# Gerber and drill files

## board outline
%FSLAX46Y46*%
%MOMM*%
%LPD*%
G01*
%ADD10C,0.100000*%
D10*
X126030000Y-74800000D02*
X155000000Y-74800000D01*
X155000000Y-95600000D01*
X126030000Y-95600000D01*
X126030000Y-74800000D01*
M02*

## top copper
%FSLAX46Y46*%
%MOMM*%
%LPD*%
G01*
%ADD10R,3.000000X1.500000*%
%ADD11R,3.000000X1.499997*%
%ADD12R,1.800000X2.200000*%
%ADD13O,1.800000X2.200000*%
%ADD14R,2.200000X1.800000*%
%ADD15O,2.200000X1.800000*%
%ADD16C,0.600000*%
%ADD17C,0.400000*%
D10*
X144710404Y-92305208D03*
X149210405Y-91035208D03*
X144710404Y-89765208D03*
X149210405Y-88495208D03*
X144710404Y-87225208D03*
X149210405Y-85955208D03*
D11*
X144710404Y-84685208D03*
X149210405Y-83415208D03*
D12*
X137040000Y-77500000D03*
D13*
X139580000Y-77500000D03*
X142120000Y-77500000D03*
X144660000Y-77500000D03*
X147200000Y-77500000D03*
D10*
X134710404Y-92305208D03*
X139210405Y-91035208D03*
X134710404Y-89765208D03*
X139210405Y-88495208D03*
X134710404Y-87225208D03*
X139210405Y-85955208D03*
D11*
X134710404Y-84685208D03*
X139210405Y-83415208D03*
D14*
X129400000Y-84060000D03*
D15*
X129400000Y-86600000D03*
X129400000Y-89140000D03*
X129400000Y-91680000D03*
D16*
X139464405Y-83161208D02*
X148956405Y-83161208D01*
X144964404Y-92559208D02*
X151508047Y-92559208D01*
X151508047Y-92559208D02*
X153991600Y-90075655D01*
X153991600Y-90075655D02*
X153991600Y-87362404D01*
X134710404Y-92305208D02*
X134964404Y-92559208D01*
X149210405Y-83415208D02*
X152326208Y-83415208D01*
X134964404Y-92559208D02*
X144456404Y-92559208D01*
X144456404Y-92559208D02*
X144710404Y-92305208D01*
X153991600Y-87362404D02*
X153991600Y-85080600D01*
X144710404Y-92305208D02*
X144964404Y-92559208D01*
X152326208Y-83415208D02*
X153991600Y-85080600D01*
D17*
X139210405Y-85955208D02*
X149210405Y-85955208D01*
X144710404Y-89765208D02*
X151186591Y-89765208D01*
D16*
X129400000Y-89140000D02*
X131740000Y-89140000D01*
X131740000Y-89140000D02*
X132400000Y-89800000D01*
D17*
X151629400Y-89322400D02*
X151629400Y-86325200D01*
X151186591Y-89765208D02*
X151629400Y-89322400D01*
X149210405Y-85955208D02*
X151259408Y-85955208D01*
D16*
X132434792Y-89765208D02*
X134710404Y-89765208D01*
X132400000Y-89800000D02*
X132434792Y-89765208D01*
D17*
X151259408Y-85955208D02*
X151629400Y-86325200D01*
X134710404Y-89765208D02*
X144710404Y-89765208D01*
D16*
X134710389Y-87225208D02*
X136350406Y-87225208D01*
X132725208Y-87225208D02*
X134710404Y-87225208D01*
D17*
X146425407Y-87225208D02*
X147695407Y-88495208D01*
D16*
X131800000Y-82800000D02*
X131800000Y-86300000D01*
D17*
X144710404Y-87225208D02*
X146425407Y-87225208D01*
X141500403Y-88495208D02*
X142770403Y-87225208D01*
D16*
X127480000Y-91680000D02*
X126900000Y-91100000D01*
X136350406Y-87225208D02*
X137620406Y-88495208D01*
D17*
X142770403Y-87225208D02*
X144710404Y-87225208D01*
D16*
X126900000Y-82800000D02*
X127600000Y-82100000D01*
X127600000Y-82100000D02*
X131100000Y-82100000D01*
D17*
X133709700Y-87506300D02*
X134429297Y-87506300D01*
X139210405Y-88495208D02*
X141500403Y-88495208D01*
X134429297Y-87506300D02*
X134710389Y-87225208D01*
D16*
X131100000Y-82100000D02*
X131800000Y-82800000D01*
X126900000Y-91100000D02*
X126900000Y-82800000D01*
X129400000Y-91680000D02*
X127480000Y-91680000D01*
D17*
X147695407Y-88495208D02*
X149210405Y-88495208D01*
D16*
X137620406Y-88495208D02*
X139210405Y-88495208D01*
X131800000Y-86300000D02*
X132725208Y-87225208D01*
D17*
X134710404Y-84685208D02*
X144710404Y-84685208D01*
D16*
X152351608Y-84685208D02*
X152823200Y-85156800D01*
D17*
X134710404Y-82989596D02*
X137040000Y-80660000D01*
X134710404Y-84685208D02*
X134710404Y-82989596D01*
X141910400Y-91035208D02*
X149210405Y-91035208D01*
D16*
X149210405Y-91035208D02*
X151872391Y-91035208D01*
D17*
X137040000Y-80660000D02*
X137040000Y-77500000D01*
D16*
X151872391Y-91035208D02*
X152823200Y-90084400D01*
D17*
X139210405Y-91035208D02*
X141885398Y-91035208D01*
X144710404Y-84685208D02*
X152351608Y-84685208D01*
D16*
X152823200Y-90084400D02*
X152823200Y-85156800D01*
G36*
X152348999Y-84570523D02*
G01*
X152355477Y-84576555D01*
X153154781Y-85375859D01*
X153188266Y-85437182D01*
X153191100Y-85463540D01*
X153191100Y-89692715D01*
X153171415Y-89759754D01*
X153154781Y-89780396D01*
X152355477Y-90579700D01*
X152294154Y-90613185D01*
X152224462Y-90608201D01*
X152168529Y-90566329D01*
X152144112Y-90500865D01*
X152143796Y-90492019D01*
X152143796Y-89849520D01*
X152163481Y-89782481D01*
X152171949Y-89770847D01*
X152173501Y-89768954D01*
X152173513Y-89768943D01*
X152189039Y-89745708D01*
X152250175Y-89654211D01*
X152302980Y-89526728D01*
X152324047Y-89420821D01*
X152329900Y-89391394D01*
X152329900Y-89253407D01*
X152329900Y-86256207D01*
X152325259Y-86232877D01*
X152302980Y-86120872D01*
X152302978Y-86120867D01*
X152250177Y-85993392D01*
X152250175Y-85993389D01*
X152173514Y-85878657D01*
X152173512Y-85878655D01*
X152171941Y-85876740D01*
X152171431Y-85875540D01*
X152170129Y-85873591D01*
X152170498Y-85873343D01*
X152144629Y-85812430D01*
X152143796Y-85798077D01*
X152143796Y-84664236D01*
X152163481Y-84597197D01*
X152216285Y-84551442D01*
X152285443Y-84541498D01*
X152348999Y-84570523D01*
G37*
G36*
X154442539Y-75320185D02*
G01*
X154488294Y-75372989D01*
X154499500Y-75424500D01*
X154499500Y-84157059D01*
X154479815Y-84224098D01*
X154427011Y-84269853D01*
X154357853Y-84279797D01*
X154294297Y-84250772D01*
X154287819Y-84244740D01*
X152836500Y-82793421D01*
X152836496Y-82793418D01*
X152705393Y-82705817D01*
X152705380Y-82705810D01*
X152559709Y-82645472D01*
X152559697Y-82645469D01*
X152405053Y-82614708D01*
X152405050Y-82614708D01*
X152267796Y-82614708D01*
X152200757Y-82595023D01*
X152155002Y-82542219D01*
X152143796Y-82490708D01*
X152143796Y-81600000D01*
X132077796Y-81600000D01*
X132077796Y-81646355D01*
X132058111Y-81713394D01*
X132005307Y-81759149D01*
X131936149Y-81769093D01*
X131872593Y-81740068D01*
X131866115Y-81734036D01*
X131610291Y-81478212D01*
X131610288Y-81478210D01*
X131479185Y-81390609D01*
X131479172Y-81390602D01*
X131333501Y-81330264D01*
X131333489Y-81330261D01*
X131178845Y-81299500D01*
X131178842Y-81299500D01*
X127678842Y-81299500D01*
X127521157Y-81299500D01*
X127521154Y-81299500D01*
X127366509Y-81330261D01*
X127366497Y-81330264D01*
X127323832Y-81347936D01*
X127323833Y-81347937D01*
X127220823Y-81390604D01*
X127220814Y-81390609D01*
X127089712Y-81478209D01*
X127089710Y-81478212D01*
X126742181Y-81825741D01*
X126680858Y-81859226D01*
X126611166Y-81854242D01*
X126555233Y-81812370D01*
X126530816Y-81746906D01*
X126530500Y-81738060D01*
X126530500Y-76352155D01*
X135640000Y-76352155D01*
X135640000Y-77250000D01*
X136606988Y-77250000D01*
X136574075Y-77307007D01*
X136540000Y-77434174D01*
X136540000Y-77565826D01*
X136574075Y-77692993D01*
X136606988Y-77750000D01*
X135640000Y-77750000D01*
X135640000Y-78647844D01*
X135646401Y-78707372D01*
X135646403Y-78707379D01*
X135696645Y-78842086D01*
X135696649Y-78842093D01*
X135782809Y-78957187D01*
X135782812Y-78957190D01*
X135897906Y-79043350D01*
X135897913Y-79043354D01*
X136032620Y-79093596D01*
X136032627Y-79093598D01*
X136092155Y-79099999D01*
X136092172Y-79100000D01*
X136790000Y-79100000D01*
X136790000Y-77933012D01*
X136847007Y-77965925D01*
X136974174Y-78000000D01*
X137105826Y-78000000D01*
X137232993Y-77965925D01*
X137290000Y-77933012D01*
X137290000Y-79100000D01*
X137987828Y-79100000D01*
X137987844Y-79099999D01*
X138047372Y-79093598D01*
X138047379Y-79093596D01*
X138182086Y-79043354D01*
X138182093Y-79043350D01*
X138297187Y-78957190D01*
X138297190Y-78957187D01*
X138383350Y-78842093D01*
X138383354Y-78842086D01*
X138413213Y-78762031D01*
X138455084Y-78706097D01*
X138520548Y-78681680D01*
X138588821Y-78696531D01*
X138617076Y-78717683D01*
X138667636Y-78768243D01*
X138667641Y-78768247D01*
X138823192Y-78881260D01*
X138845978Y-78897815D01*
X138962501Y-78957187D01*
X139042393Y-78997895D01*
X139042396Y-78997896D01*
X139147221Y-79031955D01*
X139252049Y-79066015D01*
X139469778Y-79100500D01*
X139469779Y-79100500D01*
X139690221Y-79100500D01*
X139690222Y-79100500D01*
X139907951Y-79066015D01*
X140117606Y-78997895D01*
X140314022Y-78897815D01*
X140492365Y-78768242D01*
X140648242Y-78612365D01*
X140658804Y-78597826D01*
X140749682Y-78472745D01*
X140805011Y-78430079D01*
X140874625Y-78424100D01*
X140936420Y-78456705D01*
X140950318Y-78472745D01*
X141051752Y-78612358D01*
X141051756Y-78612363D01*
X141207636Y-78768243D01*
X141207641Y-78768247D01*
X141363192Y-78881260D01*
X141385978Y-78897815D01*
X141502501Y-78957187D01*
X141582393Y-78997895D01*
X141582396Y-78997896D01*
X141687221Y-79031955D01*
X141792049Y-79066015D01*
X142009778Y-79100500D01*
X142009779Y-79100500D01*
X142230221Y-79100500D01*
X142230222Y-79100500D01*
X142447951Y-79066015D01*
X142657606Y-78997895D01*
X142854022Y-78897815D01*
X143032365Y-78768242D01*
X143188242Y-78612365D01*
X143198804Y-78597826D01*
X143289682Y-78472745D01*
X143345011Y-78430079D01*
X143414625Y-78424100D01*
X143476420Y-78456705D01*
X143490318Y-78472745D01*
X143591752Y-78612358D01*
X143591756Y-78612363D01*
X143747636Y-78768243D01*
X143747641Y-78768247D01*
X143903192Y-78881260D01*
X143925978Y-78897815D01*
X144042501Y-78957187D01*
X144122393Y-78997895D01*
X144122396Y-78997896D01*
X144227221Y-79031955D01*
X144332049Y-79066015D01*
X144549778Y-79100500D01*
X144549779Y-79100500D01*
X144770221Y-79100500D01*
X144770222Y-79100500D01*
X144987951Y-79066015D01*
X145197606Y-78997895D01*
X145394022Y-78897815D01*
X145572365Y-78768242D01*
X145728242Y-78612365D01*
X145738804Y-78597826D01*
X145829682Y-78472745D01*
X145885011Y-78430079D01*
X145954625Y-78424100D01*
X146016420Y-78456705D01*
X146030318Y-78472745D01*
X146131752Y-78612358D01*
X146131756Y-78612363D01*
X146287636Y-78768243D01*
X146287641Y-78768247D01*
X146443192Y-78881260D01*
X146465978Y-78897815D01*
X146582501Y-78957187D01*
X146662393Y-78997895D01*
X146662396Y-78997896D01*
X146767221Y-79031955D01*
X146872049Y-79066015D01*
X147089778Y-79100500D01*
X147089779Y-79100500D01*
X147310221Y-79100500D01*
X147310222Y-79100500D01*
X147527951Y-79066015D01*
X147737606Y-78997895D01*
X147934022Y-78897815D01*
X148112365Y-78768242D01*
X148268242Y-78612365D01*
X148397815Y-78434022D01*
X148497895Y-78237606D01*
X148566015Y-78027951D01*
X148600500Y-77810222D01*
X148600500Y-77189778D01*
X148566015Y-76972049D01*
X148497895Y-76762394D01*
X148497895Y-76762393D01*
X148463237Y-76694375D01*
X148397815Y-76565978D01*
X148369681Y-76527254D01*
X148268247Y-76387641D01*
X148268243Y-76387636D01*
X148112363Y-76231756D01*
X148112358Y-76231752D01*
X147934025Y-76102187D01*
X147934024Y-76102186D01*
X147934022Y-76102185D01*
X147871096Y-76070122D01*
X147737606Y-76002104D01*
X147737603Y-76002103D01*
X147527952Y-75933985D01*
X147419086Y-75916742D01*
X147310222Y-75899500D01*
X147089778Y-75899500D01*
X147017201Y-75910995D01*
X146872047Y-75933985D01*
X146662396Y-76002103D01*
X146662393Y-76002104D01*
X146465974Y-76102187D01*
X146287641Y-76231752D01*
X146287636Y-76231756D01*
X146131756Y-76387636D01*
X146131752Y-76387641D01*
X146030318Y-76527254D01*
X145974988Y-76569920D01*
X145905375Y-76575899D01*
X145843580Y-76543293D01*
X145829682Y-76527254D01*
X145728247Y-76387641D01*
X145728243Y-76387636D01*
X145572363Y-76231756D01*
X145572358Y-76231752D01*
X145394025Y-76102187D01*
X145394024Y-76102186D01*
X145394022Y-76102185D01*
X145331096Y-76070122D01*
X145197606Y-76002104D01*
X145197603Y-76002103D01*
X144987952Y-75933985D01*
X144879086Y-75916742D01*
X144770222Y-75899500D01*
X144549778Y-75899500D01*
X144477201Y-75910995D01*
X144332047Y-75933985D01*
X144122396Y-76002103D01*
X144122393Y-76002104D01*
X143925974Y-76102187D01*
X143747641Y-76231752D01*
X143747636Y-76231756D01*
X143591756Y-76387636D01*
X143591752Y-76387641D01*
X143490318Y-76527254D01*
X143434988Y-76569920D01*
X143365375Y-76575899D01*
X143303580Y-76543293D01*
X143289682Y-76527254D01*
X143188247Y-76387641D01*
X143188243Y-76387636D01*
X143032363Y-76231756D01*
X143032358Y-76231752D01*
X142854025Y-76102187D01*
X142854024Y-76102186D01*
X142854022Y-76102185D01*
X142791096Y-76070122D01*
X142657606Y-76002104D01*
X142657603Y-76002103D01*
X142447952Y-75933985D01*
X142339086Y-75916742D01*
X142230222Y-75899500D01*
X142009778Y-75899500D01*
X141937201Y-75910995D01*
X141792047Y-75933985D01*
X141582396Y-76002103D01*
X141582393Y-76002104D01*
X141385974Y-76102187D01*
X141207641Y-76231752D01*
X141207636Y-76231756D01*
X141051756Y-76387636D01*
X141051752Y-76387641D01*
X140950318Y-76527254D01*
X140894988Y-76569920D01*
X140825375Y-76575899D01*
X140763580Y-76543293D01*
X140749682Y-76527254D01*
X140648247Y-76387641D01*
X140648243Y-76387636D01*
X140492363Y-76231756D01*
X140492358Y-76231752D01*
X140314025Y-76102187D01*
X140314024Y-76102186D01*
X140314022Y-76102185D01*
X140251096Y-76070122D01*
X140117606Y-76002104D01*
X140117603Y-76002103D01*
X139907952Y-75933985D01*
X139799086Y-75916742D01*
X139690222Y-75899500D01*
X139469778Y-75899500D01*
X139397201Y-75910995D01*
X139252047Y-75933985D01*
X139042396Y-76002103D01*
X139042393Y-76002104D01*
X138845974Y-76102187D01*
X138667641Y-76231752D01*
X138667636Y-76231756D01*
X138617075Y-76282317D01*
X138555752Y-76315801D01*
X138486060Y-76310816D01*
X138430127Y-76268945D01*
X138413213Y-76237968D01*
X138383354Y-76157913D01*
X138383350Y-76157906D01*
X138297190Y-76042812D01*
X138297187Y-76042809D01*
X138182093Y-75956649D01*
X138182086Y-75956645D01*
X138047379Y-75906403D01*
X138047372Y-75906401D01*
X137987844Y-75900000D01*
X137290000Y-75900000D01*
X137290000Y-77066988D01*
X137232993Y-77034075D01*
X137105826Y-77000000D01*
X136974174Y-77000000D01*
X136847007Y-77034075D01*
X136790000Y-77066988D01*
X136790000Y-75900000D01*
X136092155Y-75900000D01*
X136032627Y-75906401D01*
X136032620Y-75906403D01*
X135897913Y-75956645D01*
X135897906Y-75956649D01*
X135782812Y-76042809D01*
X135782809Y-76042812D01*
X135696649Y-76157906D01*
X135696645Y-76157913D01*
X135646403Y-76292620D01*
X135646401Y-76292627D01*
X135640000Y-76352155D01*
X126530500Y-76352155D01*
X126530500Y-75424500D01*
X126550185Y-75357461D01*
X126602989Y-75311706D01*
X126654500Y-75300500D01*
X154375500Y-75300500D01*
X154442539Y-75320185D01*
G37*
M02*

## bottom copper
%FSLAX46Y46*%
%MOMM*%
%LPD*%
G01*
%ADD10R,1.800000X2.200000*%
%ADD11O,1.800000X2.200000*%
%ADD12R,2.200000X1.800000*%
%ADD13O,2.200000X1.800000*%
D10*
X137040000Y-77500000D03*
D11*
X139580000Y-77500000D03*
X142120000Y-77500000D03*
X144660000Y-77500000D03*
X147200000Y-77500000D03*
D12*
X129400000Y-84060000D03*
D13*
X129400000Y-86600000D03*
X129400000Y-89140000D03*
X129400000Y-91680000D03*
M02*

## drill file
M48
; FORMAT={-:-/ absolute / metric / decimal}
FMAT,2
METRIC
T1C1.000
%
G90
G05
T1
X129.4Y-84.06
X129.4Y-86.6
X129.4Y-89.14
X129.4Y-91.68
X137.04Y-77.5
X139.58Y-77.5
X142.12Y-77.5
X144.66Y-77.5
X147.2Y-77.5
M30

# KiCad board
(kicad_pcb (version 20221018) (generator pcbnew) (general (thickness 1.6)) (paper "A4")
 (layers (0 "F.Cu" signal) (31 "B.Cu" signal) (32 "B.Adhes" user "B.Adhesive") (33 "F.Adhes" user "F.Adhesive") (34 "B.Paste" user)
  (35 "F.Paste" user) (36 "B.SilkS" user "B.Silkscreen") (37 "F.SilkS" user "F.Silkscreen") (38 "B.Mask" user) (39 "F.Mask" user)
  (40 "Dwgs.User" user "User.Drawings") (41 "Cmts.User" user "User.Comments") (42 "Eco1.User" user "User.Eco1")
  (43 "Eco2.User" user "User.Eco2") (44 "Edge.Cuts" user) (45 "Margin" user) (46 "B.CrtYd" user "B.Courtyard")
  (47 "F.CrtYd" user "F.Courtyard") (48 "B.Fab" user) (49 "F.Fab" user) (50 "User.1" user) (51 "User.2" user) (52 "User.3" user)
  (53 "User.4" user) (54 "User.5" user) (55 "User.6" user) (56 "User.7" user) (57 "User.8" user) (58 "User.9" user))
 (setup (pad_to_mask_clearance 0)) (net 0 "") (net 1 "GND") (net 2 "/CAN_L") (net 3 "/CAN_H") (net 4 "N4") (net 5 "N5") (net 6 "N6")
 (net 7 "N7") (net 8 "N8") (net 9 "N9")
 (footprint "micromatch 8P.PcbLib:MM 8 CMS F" (layer "F.Cu") (at 144.710404 92.305208 -90)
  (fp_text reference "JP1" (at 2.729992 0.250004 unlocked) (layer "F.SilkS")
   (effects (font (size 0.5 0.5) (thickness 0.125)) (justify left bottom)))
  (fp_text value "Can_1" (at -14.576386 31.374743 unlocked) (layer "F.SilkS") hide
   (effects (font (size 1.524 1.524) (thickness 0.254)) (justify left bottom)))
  (pad "1" smd rect (at 0 0 270) (size 1.5 3) (layers "F.Cu" "F.Paste" "F.Mask"))
  (pad "2" smd rect (at -1.27 -4.500001 270) (size 1.5 3) (layers "F.Cu" "F.Paste" "F.Mask") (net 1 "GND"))
  (pad "3" smd rect (at -2.54 0 270) (size 1.5 3) (layers "F.Cu" "F.Paste" "F.Mask") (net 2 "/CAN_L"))
  (pad "4" smd rect (at -3.81 -4.500001 270) (size 1.5 3) (layers "F.Cu" "F.Paste" "F.Mask") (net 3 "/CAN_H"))
  (pad "5" smd rect (at -5.08 0 270) (size 1.5 3) (layers "F.Cu" "F.Paste" "F.Mask") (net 3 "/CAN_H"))
  (pad "6" smd rect (at -6.35 -4.500001 270) (size 1.5 3) (layers "F.Cu" "F.Paste" "F.Mask") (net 2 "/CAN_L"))
  (pad "7" smd rect (at -7.62 0 270) (size 1.499997 3) (layers "F.Cu" "F.Paste" "F.Mask") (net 1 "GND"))
  (pad "8" smd rect (at -8.89 -4.500001 270) (size 1.499997 3) (layers "F.Cu" "F.Paste" "F.Mask")))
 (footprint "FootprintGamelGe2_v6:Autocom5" (layer "F.Cu") (at 137.04 77.5 90)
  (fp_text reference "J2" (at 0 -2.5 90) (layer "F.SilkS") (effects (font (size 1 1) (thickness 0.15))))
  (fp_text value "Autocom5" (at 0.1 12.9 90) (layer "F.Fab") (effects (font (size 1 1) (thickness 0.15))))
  (pad "1" thru_hole rect (at 0 0 90) (size 2.2 1.8) (drill 1) (layers "*.Cu" "*.Mask") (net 1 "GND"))
  (pad "2" thru_hole oval (at 0 2.54 90) (size 2.2 1.8) (drill 1) (layers "*.Cu" "*.Mask") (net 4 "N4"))
  (pad "3" thru_hole oval (at 0 5.08 90) (size 2.2 1.8) (drill 1) (layers "*.Cu" "*.Mask") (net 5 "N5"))
  (pad "4" thru_hole oval (at 0 7.62 90) (size 2.2 1.8) (drill 1) (layers "*.Cu" "*.Mask") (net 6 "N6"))
  (pad "5" thru_hole oval (at 0 10.16 90) (size 2.2 1.8) (drill 1) (layers "*.Cu" "*.Mask") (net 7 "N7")))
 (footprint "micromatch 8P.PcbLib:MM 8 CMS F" (layer "F.Cu") (at 134.710404 92.305208 -90)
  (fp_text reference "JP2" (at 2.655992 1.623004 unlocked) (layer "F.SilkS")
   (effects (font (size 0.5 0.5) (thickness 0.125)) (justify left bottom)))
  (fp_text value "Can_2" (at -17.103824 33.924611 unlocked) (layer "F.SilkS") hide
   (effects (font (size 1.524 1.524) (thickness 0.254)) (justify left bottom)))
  (pad "1" smd rect (at 0 0 270) (size 1.5 3) (layers "F.Cu" "F.Paste" "F.Mask"))
  (pad "2" smd rect (at -1.27 -4.500001 270) (size 1.5 3) (layers "F.Cu" "F.Paste" "F.Mask") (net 1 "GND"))
  (pad "3" smd rect (at -2.54 0 270) (size 1.5 3) (layers "F.Cu" "F.Paste" "F.Mask") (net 2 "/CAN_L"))
  (pad "4" smd rect (at -3.81 -4.500001 270) (size 1.5 3) (layers "F.Cu" "F.Paste" "F.Mask") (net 3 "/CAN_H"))
  (pad "5" smd rect (at -5.08 0 270) (size 1.5 3) (layers "F.Cu" "F.Paste" "F.Mask") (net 3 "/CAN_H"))
  (pad "6" smd rect (at -6.35 -4.500001 270) (size 1.5 3) (layers "F.Cu" "F.Paste" "F.Mask") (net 2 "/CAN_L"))
  (pad "7" smd rect (at -7.62 0 270) (size 1.499997 3) (layers "F.Cu" "F.Paste" "F.Mask") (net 1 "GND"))
  (pad "8" smd rect (at -8.89 -4.500001 270) (size 1.499997 3) (layers "F.Cu" "F.Paste" "F.Mask")))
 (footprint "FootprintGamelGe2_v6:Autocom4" (layer "B.Cu") (at 129.4 84.06 180)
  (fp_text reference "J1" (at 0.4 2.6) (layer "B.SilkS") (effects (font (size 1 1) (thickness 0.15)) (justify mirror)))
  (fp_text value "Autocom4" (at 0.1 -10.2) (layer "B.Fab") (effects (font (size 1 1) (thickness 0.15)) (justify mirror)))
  (pad "1" thru_hole rect (at 0 0 180) (size 2.2 1.8) (drill 1) (layers "*.Cu" "*.Mask") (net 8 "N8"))
  (pad "2" thru_hole oval (at 0 -2.54 180) (size 2.2 1.8) (drill 1) (layers "*.Cu" "*.Mask") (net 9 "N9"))
  (pad "3" thru_hole oval (at 0 -5.08 180) (size 2.2 1.8) (drill 1) (layers "*.Cu" "*.Mask") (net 2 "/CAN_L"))
  (pad "4" thru_hole oval (at 0 -7.62 180) (size 2.2 1.8) (drill 1) (layers "*.Cu" "*.Mask") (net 3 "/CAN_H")))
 (gr_rect (start 126.03 74.8) (end 155 95.6) (stroke (width 0.1) (type default)) (fill none) (layer "Edge.Cuts"))
 (segment (start 139.464405 83.161208) (end 148.956405 83.161208) (width 0.6) (layer "F.Cu") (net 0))
 (segment (start 144.964404 92.559208) (end 151.508047 92.559208) (width 0.6) (layer "F.Cu") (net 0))
 (segment (start 151.508047 92.559208) (end 153.9916 90.075655) (width 0.6) (layer "F.Cu") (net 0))
 (segment (start 153.9916 90.075655) (end 153.9916 87.362404) (width 0.6) (layer "F.Cu") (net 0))
 (segment (start 134.710404 92.305208) (end 134.964404 92.559208) (width 0.6) (layer "F.Cu") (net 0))
 (segment (start 149.210405 83.415208) (end 152.326208 83.415208) (width 0.6) (layer "F.Cu") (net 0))
 (segment (start 134.964404 92.559208) (end 144.456404 92.559208) (width 0.6) (layer "F.Cu") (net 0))
 (segment (start 144.456404 92.559208) (end 144.710404 92.305208) (width 0.6) (layer "F.Cu") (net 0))
 (segment (start 153.9916 87.362404) (end 153.9916 85.0806) (width 0.6) (layer "F.Cu") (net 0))
 (segment (start 144.710404 92.305208) (end 144.964404 92.559208) (width 0.6) (layer "F.Cu") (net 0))
 (segment (start 152.326208 83.415208) (end 153.9916 85.0806) (width 0.6) (layer "F.Cu") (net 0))
 (segment (start 139.210405 85.955208) (end 149.210405 85.955208) (width 0.4) (layer "F.Cu") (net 2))
 (segment (start 144.710404 89.765208) (end 151.186591 89.765208) (width 0.4) (layer "F.Cu") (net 2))
 (segment (start 129.4 89.14) (end 131.74 89.14) (width 0.6) (layer "F.Cu") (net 2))
 (segment (start 131.74 89.14) (end 132.4 89.8) (width 0.6) (layer "F.Cu") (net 2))
 (segment (start 151.6294 89.3224) (end 151.6294 86.3252) (width 0.4) (layer "F.Cu") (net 2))
 (segment (start 151.186591 89.765208) (end 151.6294 89.3224) (width 0.4) (layer "F.Cu") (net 2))
 (segment (start 149.210405 85.955208) (end 151.259408 85.955208) (width 0.4) (layer "F.Cu") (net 2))
 (segment (start 132.434792 89.765208) (end 134.710404 89.765208) (width 0.6) (layer "F.Cu") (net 2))
 (segment (start 132.4 89.8) (end 132.434792 89.765208) (width 0.6) (layer "F.Cu") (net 2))
 (segment (start 151.259408 85.955208) (end 151.6294 86.3252) (width 0.4) (layer "F.Cu") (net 2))
 (segment (start 134.710404 89.765208) (end 144.710404 89.765208) (width 0.4) (layer "F.Cu") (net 2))
 (segment (start 134.710389 87.225208) (end 136.350406 87.225208) (width 0.6) (layer "F.Cu") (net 3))
 (segment (start 132.725208 87.225208) (end 134.710404 87.225208) (width 0.6) (layer "F.Cu") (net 3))
 (segment (start 146.425407 87.225208) (end 147.695407 88.495208) (width 0.4) (layer "F.Cu") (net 3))
 (segment (start 131.8 82.8) (end 131.8 86.3) (width 0.6) (layer "F.Cu") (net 3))
 (segment (start 144.710404 87.225208) (end 146.425407 87.225208) (width 0.4) (layer "F.Cu") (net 3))
 (segment (start 141.500403 88.495208) (end 142.770403 87.225208) (width 0.4) (layer "F.Cu") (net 3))
 (segment (start 127.48 91.68) (end 126.9 91.1) (width 0.6) (layer "F.Cu") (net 3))
 (segment (start 136.350406 87.225208) (end 137.620406 88.495208) (width 0.6) (layer "F.Cu") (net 3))
 (segment (start 142.770403 87.225208) (end 144.710404 87.225208) (width 0.4) (layer "F.Cu") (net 3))
 (segment (start 126.9 82.8) (end 127.6 82.1) (width 0.6) (layer "F.Cu") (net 3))
 (segment (start 127.6 82.1) (end 131.1 82.1) (width 0.6) (layer "F.Cu") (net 3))
 (segment (start 133.7097 87.5063) (end 134.429297 87.5063) (width 0.4) (layer "F.Cu") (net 3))
 (segment (start 139.210405 88.495208) (end 141.500403 88.495208) (width 0.4) (layer "F.Cu") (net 3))
 (segment (start 134.429297 87.5063) (end 134.710389 87.225208) (width 0.4) (layer "F.Cu") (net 3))
 (segment (start 131.1 82.1) (end 131.8 82.8) (width 0.6) (layer "F.Cu") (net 3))
 (segment (start 126.9 91.1) (end 126.9 82.8) (width 0.6) (layer "F.Cu") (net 3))
 (segment (start 129.4 91.68) (end 127.48 91.68) (width 0.6) (layer "F.Cu") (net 3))
 (segment (start 147.695407 88.495208) (end 149.210405 88.495208) (width 0.4) (layer "F.Cu") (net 3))
 (segment (start 137.620406 88.495208) (end 139.210405 88.495208) (width 0.6) (layer "F.Cu") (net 3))
 (segment (start 131.8 86.3) (end 132.725208 87.225208) (width 0.6) (layer "F.Cu") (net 3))
 (segment (start 134.710404 84.685208) (end 144.710404 84.685208) (width 0.4) (layer "F.Cu") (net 1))
 (segment (start 152.351608 84.685208) (end 152.8232 85.1568) (width 0.6) (layer "F.Cu") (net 1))
 (segment (start 134.710404 82.989596) (end 137.04 80.66) (width 0.4) (layer "F.Cu") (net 1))
 (segment (start 134.710404 84.685208) (end 134.710404 82.989596) (width 0.4) (layer "F.Cu") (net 1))
 (segment (start 141.9104 91.035208) (end 149.210405 91.035208) (width 0.4) (layer "F.Cu") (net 1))
 (segment (start 149.210405 91.035208) (end 151.872391 91.035208) (width 0.6) (layer "F.Cu") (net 1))
 (segment (start 137.04 80.66) (end 137.04 77.5) (width 0.4) (layer "F.Cu") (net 1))
 (segment (start 151.872391 91.035208) (end 152.8232 90.0844) (width 0.6) (layer "F.Cu") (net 1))
 (segment (start 139.210405 91.035208) (end 141.885398 91.035208) (width 0.4) (layer "F.Cu") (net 1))
 (segment (start 144.710404 84.685208) (end 152.351608 84.685208) (width 0.4) (layer "F.Cu") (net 1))
 (segment (start 152.8232 90.0844) (end 152.8232 85.1568) (width 0.6) (layer "F.Cu") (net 1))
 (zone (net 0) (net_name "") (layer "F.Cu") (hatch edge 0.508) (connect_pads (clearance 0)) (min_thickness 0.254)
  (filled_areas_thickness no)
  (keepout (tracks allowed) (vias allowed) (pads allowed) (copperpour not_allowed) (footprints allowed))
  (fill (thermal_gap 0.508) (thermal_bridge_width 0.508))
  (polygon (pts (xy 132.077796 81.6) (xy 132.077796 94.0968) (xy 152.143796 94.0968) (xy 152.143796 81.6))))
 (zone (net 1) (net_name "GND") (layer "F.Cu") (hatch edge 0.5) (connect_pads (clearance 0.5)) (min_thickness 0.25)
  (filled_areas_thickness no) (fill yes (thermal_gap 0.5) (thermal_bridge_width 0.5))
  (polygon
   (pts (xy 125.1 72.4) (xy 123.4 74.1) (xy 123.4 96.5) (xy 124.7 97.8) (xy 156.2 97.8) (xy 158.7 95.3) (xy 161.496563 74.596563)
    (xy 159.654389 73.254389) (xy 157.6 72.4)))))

